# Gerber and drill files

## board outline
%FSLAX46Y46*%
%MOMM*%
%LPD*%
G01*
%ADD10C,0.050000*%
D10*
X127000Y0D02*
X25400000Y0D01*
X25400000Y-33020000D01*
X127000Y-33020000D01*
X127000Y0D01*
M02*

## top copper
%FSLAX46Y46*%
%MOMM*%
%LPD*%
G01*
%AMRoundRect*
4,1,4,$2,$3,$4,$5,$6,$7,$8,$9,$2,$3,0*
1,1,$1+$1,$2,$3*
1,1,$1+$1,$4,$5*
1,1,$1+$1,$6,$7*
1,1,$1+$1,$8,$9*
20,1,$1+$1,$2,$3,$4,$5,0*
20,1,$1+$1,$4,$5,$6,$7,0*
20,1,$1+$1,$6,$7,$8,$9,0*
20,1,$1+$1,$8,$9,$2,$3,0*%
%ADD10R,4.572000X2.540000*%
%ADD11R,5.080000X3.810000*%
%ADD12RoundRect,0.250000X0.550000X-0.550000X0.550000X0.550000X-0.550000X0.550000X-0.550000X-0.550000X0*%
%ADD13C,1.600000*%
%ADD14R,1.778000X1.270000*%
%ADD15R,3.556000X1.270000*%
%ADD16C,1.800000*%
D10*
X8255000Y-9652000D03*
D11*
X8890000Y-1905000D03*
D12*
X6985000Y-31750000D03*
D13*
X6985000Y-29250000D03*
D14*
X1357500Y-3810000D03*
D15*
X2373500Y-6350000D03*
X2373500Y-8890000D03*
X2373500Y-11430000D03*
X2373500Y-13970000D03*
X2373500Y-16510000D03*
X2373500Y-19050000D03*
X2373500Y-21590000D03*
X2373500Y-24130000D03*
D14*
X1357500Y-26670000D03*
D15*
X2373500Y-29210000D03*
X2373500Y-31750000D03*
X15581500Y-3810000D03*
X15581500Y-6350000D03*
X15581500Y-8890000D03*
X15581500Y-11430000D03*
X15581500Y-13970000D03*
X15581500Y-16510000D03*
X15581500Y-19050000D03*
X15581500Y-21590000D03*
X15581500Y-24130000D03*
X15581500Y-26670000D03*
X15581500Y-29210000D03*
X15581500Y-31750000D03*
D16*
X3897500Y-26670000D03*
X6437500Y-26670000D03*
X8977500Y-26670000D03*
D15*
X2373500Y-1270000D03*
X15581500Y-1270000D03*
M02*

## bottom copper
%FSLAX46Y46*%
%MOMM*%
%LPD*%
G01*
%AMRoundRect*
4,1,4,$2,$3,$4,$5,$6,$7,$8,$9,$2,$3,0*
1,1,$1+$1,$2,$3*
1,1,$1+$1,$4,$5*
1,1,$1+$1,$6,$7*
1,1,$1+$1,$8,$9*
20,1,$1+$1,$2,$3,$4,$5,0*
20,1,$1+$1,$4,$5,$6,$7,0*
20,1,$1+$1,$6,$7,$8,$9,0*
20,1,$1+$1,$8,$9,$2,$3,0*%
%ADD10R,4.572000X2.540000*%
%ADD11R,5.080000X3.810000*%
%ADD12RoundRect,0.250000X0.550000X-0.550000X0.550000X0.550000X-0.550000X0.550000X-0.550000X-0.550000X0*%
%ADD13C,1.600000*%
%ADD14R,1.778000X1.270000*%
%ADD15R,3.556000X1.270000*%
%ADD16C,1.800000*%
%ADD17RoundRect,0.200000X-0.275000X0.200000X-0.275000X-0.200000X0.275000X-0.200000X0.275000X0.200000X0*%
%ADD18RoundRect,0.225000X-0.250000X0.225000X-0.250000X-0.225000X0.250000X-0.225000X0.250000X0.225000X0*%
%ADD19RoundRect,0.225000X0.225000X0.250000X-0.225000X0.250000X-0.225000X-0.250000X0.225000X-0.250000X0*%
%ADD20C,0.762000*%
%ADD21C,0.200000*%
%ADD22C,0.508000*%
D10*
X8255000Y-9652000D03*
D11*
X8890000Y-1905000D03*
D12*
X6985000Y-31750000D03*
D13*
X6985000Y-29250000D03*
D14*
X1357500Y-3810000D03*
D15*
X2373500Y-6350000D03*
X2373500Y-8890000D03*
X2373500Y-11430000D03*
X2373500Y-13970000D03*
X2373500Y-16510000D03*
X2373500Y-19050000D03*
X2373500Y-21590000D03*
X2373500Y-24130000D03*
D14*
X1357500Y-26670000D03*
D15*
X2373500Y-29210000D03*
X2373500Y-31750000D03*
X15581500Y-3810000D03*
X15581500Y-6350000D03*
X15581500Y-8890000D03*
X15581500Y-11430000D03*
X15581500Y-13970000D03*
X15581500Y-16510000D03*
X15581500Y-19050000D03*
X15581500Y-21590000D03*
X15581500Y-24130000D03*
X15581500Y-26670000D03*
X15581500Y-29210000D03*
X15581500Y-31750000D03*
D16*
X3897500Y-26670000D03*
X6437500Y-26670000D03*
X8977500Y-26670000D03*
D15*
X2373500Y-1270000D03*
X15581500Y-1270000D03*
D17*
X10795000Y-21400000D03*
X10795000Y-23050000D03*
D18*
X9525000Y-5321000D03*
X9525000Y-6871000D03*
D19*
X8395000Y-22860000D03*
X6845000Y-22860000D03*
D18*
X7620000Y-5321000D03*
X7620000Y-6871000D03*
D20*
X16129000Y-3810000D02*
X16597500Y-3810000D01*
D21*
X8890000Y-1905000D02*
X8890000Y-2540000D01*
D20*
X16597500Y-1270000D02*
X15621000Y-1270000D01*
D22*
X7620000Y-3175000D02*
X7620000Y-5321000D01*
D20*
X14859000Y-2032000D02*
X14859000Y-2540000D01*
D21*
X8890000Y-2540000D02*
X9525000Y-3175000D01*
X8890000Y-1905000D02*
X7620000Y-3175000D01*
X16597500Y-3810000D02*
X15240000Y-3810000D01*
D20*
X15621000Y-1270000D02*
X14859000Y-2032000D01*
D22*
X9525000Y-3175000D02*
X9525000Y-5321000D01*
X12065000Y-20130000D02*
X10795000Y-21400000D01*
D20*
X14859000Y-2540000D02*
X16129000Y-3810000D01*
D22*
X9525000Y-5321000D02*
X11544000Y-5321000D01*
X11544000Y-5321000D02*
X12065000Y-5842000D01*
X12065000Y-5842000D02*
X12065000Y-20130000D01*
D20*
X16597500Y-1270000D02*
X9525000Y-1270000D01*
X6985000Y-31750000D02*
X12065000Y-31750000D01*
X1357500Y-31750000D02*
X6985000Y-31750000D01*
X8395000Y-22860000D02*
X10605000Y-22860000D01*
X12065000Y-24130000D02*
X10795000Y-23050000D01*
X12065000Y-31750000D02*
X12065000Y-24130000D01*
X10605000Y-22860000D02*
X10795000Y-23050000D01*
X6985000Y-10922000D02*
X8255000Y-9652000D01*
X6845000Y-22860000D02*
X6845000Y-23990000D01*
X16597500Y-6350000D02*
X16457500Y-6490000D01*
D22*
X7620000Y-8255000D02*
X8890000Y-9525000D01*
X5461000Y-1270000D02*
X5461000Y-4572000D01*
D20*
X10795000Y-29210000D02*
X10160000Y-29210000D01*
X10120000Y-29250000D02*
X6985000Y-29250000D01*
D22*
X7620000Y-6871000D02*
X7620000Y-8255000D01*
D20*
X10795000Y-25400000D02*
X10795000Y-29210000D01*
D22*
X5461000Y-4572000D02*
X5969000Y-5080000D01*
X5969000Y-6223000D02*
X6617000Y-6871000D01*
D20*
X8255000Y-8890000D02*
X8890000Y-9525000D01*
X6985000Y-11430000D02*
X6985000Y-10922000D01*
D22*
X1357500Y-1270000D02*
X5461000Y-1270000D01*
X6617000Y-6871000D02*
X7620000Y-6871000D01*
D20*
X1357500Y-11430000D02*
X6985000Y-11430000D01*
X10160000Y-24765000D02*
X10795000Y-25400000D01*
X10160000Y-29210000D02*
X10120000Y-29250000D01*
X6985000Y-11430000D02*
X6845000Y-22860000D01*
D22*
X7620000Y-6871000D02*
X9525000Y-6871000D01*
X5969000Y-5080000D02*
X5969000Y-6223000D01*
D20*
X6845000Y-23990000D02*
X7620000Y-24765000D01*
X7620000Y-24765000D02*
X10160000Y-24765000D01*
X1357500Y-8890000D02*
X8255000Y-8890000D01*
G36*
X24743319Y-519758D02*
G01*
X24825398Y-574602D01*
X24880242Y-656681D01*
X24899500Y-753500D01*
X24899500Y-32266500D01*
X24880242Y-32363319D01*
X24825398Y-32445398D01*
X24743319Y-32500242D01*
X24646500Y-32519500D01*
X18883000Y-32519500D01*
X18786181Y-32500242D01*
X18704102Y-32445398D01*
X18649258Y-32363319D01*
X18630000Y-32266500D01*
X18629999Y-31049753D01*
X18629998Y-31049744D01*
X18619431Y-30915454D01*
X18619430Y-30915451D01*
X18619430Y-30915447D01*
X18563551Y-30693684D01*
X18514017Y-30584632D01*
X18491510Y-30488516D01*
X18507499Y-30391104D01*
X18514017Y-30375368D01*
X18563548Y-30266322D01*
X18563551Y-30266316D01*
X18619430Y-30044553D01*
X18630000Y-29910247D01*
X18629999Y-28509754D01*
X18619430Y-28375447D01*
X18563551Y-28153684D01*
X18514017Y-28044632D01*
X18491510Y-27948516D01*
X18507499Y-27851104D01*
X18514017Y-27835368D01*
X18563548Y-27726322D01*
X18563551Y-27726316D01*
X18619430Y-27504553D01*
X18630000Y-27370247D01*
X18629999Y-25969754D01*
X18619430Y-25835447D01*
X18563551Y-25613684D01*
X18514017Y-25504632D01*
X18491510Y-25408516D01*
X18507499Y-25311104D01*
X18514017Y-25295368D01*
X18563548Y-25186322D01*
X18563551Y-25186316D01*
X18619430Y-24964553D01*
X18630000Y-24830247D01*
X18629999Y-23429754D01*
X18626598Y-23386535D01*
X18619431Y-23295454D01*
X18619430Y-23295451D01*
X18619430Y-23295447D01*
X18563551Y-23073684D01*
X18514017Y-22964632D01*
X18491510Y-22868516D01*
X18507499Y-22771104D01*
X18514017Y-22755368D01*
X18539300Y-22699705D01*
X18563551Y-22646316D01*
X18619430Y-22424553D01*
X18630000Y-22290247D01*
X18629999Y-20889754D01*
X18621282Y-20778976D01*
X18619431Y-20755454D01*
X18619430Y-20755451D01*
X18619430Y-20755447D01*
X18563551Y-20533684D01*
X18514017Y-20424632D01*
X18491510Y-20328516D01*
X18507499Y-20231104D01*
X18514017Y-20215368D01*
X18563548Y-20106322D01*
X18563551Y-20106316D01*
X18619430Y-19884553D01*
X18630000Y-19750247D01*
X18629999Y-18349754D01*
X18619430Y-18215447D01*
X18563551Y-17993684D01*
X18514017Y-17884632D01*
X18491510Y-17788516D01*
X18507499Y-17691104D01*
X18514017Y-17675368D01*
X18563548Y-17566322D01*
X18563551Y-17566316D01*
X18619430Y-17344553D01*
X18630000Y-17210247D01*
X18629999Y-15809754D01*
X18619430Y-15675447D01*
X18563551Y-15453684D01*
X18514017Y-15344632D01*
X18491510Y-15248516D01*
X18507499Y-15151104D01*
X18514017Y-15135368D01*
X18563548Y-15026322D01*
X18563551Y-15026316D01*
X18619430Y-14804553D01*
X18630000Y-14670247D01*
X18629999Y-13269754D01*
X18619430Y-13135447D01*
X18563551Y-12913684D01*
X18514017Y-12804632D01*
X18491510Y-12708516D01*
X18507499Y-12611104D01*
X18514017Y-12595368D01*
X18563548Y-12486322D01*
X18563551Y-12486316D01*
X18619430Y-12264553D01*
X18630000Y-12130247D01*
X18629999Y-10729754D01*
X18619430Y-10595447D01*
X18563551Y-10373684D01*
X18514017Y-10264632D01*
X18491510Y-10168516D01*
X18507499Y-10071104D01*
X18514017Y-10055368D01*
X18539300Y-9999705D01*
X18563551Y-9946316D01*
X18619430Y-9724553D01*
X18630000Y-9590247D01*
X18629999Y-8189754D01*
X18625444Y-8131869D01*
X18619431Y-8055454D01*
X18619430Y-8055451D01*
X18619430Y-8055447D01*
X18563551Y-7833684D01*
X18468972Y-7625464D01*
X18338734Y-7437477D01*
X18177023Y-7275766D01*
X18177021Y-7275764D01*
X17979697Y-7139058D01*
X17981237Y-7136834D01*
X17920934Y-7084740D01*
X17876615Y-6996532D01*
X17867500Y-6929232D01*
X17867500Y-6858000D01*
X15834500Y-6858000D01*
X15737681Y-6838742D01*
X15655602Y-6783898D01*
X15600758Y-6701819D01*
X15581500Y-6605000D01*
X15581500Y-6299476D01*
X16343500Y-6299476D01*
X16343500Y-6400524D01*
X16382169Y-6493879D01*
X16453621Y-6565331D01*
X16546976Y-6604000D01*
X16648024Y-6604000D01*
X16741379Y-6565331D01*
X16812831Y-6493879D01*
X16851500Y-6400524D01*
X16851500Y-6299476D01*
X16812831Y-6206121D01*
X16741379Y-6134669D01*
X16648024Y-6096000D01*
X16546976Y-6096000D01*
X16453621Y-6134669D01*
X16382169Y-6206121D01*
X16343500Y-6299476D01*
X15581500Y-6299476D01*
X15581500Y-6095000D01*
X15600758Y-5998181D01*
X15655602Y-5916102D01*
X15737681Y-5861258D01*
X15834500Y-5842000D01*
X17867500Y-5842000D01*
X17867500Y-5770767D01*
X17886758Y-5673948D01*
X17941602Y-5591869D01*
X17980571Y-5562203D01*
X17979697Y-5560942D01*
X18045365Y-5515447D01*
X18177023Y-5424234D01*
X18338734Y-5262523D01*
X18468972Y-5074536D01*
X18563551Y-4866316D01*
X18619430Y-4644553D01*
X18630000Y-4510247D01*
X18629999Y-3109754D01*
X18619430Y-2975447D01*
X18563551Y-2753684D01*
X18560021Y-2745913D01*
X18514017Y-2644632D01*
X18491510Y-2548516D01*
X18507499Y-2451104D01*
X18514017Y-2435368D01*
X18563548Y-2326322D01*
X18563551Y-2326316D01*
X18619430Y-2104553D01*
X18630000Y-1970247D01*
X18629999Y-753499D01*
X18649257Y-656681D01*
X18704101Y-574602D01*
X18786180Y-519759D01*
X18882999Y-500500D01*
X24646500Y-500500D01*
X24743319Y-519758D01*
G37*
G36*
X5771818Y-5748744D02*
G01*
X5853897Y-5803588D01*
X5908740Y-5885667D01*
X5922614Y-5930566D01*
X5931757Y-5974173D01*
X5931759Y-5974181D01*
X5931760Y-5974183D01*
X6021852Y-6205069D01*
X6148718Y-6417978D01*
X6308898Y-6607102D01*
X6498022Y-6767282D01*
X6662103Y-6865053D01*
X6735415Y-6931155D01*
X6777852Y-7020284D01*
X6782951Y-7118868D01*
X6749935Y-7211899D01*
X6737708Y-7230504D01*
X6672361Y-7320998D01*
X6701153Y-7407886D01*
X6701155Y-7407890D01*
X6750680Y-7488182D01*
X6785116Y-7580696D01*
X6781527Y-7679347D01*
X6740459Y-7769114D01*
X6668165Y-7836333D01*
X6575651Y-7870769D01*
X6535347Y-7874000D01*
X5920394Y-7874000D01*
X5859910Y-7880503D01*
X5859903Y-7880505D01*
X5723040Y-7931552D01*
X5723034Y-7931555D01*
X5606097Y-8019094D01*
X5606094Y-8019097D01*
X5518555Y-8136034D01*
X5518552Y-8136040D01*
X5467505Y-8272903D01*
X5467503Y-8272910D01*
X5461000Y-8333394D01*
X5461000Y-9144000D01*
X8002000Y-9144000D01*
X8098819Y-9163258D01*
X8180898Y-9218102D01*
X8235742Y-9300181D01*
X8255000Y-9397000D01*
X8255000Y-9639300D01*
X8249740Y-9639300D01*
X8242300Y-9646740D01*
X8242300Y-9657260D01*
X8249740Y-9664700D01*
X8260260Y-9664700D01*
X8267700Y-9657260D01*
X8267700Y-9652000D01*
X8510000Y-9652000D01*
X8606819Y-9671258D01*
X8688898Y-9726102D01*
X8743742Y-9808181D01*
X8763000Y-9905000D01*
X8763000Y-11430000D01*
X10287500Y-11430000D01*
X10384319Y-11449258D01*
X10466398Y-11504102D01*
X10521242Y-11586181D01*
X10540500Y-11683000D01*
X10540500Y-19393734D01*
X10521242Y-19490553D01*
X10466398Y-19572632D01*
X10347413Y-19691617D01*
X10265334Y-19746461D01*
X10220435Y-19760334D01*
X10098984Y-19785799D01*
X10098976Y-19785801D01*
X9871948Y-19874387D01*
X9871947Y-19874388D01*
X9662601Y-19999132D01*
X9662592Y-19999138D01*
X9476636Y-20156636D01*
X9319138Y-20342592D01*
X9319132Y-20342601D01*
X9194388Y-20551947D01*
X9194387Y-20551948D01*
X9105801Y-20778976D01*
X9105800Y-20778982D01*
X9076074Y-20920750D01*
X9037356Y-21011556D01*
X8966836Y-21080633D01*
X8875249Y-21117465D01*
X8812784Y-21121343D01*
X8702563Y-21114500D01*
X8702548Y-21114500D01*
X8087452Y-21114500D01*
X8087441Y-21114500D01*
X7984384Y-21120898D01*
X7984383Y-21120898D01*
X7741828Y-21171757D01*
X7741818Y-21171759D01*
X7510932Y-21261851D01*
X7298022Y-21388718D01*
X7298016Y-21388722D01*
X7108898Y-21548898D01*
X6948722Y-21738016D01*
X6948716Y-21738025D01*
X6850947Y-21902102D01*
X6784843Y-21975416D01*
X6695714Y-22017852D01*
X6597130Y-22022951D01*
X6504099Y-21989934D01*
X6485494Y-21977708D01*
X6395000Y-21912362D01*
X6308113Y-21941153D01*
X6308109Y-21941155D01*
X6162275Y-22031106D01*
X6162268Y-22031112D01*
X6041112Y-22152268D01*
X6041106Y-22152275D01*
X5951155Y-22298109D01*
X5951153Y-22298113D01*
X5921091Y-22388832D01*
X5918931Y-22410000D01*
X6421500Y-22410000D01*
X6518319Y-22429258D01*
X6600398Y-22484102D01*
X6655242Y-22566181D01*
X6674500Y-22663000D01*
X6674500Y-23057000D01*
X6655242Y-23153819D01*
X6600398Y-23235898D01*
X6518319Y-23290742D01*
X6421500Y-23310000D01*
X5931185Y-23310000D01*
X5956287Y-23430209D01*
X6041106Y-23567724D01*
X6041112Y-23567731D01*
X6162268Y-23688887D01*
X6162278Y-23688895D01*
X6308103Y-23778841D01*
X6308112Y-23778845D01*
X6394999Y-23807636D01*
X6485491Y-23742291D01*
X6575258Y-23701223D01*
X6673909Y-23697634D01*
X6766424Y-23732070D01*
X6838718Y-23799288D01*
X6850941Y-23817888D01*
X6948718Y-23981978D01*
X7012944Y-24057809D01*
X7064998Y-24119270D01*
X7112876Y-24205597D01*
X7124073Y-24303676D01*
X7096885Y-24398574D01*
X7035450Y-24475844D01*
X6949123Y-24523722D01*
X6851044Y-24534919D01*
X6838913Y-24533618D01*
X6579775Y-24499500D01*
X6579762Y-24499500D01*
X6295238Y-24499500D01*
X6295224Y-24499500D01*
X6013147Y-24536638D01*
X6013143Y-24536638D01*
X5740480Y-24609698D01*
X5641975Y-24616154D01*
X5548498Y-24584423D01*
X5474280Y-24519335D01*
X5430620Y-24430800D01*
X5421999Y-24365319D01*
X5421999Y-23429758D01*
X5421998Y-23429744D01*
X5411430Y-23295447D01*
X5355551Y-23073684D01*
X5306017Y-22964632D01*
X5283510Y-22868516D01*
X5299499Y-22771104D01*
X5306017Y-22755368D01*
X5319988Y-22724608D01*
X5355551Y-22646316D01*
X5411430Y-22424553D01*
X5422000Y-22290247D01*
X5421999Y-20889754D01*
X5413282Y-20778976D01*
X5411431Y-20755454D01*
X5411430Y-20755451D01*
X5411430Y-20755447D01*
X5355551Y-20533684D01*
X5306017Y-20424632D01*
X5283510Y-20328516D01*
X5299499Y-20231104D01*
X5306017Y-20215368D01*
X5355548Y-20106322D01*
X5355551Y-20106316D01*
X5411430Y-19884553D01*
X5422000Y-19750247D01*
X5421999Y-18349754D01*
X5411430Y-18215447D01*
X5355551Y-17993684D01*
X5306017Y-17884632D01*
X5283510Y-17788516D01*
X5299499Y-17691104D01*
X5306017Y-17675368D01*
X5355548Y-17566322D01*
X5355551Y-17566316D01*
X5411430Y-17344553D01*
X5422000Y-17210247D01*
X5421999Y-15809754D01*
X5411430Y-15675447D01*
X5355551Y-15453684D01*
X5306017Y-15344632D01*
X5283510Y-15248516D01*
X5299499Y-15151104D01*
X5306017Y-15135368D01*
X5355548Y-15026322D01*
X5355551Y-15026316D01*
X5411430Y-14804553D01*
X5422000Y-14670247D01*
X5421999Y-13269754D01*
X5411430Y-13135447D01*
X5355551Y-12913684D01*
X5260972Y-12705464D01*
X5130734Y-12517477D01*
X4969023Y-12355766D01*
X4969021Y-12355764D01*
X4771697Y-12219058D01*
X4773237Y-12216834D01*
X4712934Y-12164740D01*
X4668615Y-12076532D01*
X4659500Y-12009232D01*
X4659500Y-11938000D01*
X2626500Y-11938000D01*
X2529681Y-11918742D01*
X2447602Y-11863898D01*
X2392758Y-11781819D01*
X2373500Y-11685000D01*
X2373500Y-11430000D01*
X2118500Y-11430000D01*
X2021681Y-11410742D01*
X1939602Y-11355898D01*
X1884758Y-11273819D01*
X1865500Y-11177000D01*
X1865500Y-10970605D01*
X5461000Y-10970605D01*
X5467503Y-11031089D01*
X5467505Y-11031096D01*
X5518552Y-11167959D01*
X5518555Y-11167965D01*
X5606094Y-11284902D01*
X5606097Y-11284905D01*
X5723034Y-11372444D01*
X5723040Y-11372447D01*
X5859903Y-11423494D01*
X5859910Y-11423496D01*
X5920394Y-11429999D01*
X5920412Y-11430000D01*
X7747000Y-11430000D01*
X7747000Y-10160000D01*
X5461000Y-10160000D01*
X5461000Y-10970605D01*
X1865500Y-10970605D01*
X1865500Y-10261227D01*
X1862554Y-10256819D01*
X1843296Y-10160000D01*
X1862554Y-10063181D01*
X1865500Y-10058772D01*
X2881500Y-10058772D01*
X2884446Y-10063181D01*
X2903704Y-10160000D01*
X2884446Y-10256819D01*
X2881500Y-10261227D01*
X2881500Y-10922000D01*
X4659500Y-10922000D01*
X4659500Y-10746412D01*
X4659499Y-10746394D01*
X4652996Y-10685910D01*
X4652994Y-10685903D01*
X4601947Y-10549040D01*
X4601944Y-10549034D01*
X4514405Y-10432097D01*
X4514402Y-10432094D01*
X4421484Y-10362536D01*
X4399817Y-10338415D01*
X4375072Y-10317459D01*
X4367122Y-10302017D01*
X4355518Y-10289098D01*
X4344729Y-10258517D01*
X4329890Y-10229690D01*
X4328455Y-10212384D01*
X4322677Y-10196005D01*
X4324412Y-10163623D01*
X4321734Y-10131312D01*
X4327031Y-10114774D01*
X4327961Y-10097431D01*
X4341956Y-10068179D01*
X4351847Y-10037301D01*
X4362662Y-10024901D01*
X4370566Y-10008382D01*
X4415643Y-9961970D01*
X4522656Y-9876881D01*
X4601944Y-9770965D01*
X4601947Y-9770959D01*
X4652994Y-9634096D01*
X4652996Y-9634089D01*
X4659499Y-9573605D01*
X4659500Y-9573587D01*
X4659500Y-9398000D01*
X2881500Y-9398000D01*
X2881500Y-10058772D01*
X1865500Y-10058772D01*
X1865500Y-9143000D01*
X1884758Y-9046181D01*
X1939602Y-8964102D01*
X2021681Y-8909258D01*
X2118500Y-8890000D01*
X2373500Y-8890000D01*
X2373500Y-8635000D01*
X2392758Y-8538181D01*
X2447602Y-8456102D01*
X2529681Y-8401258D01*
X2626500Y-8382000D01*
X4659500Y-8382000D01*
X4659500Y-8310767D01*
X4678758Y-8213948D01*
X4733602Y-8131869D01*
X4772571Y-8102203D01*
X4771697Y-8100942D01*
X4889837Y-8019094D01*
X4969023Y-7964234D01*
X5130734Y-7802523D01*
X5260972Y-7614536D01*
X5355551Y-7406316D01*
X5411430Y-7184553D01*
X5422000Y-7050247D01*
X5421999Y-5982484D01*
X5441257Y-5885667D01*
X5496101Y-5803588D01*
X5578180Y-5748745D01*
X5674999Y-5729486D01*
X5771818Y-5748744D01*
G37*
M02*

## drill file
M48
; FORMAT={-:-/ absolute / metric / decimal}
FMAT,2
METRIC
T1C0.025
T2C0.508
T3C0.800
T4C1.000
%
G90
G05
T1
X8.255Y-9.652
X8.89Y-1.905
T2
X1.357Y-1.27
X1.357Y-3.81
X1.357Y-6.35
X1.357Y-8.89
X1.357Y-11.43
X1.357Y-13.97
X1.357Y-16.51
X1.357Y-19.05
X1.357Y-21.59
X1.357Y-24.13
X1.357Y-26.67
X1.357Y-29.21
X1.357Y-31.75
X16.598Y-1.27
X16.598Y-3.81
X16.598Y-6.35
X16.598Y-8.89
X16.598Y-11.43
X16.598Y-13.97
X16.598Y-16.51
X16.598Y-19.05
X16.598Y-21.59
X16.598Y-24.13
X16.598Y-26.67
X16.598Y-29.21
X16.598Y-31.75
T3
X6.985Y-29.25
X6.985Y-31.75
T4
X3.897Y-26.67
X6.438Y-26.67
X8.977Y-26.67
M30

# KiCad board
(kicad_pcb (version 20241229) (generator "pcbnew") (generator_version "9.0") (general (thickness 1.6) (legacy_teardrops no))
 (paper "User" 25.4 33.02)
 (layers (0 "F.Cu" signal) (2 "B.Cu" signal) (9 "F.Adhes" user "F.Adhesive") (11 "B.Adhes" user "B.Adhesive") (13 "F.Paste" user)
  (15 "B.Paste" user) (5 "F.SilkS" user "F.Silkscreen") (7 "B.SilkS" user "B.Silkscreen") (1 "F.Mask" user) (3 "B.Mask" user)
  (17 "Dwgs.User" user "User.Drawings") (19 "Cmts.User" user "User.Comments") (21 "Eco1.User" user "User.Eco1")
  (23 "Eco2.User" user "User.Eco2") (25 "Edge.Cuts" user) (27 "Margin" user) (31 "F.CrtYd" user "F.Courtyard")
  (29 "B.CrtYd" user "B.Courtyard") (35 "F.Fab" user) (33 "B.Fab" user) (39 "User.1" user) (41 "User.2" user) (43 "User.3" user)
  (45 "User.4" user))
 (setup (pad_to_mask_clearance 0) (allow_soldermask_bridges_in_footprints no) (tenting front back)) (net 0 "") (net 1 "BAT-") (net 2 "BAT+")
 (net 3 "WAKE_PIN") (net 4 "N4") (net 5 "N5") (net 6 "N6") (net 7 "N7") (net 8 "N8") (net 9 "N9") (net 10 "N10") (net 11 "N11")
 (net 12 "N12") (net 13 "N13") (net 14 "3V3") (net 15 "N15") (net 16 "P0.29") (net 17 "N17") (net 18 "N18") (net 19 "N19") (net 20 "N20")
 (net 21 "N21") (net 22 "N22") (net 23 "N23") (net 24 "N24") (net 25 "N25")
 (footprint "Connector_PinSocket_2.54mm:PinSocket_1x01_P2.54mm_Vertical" (layer "F.Cu") (at 8.255 9.652)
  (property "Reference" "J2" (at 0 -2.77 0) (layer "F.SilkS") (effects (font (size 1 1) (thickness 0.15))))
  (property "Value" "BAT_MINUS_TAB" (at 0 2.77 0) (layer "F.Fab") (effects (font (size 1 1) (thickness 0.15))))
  (pad "1" thru_hole rect (at 0 0) (size 4.572 2.54) (drill 0.0254) (layers "*.Cu" "*.Mask") (remove_unused_layers no) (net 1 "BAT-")))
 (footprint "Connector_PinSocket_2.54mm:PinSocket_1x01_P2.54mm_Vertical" (layer "F.Cu") (at 8.89 1.905 180)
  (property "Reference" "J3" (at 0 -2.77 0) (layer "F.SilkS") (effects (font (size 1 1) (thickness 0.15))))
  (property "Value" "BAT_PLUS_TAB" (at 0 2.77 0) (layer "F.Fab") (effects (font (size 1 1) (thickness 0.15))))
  (pad "1" thru_hole rect (at 0 0 180) (size 5.08 3.81) (drill 0.0254) (layers "*.Cu" "*.Mask") (remove_unused_layers no) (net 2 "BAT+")))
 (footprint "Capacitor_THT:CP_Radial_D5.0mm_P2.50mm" (layer "F.Cu") (at 6.985 31.75 90)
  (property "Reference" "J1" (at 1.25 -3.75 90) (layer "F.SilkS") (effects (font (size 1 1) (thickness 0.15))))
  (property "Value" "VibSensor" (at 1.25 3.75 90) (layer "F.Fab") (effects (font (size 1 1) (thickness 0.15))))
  (pad "1" thru_hole roundrect (at 0 0 90) (size 1.6 1.6) (drill 0.8) (layers "*.Cu" "*.Mask") (remove_unused_layers no)
   (roundrect_rratio 0.15625) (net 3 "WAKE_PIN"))
  (pad "2" thru_hole circle (at 2.5 0 90) (size 1.6 1.6) (drill 0.8) (layers "*.Cu" "*.Mask") (remove_unused_layers no) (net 1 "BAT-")))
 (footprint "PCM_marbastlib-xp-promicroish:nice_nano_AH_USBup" (layer "F.Cu") (at 8.9775 17.78)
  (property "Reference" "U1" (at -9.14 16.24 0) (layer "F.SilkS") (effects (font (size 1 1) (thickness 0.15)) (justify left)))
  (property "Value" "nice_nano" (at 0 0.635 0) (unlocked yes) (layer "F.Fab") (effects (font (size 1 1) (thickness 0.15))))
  (pad "1" thru_hole rect (at -7.62 -13.97) (size 1.778 1.27) (drill 0.508) (layers "*.Cu" "B.Mask") (remove_unused_layers no) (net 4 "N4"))
  (pad "2" thru_hole rect (at -7.62 -11.43) (size 3.556 1.27) (drill 0.508 (offset 1.016 0)) (layers "*.Cu" "B.Mask")
   (remove_unused_layers no) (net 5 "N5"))
  (pad "3" thru_hole rect (at -7.62 -8.89) (size 3.556 1.27) (drill 0.508 (offset 1.016 0)) (layers "*.Cu" "B.Mask")
   (remove_unused_layers no) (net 1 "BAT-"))
  (pad "4" thru_hole rect (at -7.62 -6.35) (size 3.556 1.27) (drill 0.508 (offset 1.016 0)) (layers "*.Cu" "B.Mask")
   (remove_unused_layers no) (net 1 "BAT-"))
  (pad "5" thru_hole rect (at -7.62 -3.81) (size 3.556 1.27) (drill 0.508 (offset 1.016 0)) (layers "*.Cu" "B.Mask")
   (remove_unused_layers no) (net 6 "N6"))
  (pad "6" thru_hole rect (at -7.62 -1.27) (size 3.556 1.27) (drill 0.508 (offset 1.016 0)) (layers "*.Cu" "B.Mask")
   (remove_unused_layers no) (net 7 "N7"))
  (pad "7" thru_hole rect (at -7.62 1.27) (size 3.556 1.27) (drill 0.508 (offset 1.016 0)) (layers "*.Cu" "B.Mask")
   (remove_unused_layers no) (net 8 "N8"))
  (pad "8" thru_hole rect (at -7.62 3.81) (size 3.556 1.27) (drill 0.508 (offset 1.016 0)) (layers "*.Cu" "B.Mask")
   (remove_unused_layers no) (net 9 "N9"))
  (pad "9" thru_hole rect (at -7.62 6.35) (size 3.556 1.27) (drill 0.508 (offset 1.016 0)) (layers "*.Cu" "B.Mask")
   (remove_unused_layers no) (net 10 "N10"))
  (pad "10" thru_hole rect (at -7.62 8.89) (size 1.778 1.27) (drill 0.508) (layers "*.Cu" "B.Mask") (remove_unused_layers no) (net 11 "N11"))
  (pad "11" thru_hole rect (at -7.62 11.43) (size 3.556 1.27) (drill 0.508 (offset 1.016 0)) (layers "*.Cu" "B.Mask")
   (remove_unused_layers no) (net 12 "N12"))
  (pad "12" thru_hole rect (at -7.62 13.97) (size 3.556 1.27) (drill 0.508 (offset 1.016 0)) (layers "*.Cu" "B.Mask")
   (remove_unused_layers no) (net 3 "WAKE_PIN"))
  (pad "13" thru_hole rect (at 7.62 -13.97) (size 3.556 1.27) (drill 0.508 (offset -1.016 0)) (layers "*.Cu" "B.Mask")
   (remove_unused_layers no) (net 2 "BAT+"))
  (pad "14" thru_hole rect (at 7.62 -11.43) (size 3.556 1.27) (drill 0.508 (offset -1.016 0)) (layers "*.Cu" "B.Mask")
   (remove_unused_layers no) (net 1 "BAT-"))
  (pad "15" thru_hole rect (at 7.62 -8.89) (size 3.556 1.27) (drill 0.508 (offset -1.016 0)) (layers "*.Cu" "B.Mask")
   (remove_unused_layers no) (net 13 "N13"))
  (pad "16" thru_hole rect (at 7.62 -6.35) (size 3.556 1.27) (drill 0.508 (offset -1.016 0)) (layers "*.Cu" "B.Mask")
   (remove_unused_layers no) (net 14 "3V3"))
  (pad "17" thru_hole rect (at 7.62 -3.81) (size 3.556 1.27) (drill 0.508 (offset -1.016 0)) (layers "*.Cu" "B.Mask")
   (remove_unused_layers no) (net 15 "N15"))
  (pad "18" thru_hole rect (at 7.62 -1.27) (size 3.556 1.27) (drill 0.508 (offset -1.016 0)) (layers "*.Cu" "B.Mask")
   (remove_unused_layers no) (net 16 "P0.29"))
  (pad "19" thru_hole rect (at 7.62 1.27) (size 3.556 1.27) (drill 0.508 (offset -1.016 0)) (layers "*.Cu" "B.Mask")
   (remove_unused_layers no) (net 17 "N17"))
  (pad "20" thru_hole rect (at 7.62 3.81) (size 3.556 1.27) (drill 0.508 (offset -1.016 0)) (layers "*.Cu" "B.Mask")
   (remove_unused_layers no) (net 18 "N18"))
  (pad "21" thru_hole rect (at 7.62 6.35) (size 3.556 1.27) (drill 0.508 (offset -1.016 0)) (layers "*.Cu" "B.Mask")
   (remove_unused_layers no) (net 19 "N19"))
  (pad "22" thru_hole rect (at 7.62 8.89) (size 3.556 1.27) (drill 0.508 (offset -1.016 0)) (layers "*.Cu" "B.Mask")
   (remove_unused_layers no) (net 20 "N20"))
  (pad "23" thru_hole rect (at 7.62 11.43) (size 3.556 1.27) (drill 0.508 (offset -1.016 0)) (layers "*.Cu" "B.Mask")
   (remove_unused_layers no) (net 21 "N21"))
  (pad "24" thru_hole rect (at 7.62 13.97) (size 3.556 1.27) (drill 0.508 (offset -1.016 0)) (layers "*.Cu" "B.Mask")
   (remove_unused_layers no) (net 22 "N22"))
  (pad "25" thru_hole circle (at -5.08 8.89) (size 1.8 1.8) (drill 1) (layers "*.Cu" "B.Mask") (remove_unused_layers no) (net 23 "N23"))
  (pad "26" thru_hole circle (at -2.54 8.89) (size 1.8 1.8) (drill 1) (layers "*.Cu" "B.Mask") (remove_unused_layers no) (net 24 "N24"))
  (pad "27" thru_hole circle (at 0 8.89) (size 1.8 1.8) (drill 1) (layers "*.Cu" "B.Mask") (remove_unused_layers no) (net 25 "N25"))
  (pad "28" thru_hole rect (at -7.62 -16.51) (size 3.556 1.27) (drill 0.508 (offset 1.016 0)) (layers "*.Cu" "B.Mask")
   (remove_unused_layers no) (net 1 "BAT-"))
  (pad "29" thru_hole rect (at 7.62 -16.51) (size 3.556 1.27) (drill 0.508 (offset -1.016 0)) (layers "*.Cu" "B.Mask")
   (remove_unused_layers no) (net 2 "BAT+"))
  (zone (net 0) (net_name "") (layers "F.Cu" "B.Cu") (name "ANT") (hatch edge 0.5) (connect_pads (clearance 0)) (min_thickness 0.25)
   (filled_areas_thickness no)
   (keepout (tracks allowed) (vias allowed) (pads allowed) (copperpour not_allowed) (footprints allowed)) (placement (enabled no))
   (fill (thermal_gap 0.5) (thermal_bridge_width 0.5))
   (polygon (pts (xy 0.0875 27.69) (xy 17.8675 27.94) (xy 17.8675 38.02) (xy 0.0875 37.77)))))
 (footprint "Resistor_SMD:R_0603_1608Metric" (layer "B.Cu") (at 10.795 22.225 -90)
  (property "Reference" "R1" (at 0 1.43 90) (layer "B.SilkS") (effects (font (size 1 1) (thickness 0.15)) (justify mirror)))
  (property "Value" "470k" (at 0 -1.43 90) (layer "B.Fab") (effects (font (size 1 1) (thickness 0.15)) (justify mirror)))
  (pad "1" smd roundrect (at -0.825 0 270) (size 0.8 0.95) (layers "B.Cu" "B.Mask" "B.Paste") (roundrect_rratio 0.25) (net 2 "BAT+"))
  (pad "2" smd roundrect (at 0.825 0 270) (size 0.8 0.95) (layers "B.Cu" "B.Mask" "B.Paste") (roundrect_rratio 0.25) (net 3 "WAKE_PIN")))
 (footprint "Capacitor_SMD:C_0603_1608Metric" (layer "B.Cu") (at 9.525 6.096 -90)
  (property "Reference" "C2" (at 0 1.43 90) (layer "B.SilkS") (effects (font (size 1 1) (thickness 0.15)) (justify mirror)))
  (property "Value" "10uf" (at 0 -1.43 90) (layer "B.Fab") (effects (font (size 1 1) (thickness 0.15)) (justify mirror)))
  (pad "1" smd roundrect (at -0.775 0 270) (size 0.9 0.95) (layers "B.Cu" "B.Mask" "B.Paste") (roundrect_rratio 0.25) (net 2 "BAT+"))
  (pad "2" smd roundrect (at 0.775 0 270) (size 0.9 0.95) (layers "B.Cu" "B.Mask" "B.Paste") (roundrect_rratio 0.25) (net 1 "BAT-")))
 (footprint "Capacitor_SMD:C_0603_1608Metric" (layer "B.Cu") (at 7.62 22.86 180)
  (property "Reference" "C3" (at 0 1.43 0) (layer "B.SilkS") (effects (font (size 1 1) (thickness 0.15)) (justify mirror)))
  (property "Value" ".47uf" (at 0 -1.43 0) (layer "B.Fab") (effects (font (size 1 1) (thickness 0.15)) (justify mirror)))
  (pad "1" smd roundrect (at -0.775 0 180) (size 0.9 0.95) (layers "B.Cu" "B.Mask" "B.Paste") (roundrect_rratio 0.25) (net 3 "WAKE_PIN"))
  (pad "2" smd roundrect (at 0.775 0 180) (size 0.9 0.95) (layers "B.Cu" "B.Mask" "B.Paste") (roundrect_rratio 0.25) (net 1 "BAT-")))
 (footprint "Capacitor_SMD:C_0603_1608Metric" (layer "B.Cu") (at 7.62 6.096 -90)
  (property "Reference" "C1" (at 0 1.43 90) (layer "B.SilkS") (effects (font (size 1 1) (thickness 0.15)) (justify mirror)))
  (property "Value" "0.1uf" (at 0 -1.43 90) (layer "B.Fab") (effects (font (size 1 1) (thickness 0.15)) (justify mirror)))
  (pad "1" smd roundrect (at -0.775 0 270) (size 0.9 0.95) (layers "B.Cu" "B.Mask" "B.Paste") (roundrect_rratio 0.25) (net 2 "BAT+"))
  (pad "2" smd roundrect (at 0.775 0 270) (size 0.9 0.95) (layers "B.Cu" "B.Mask" "B.Paste") (roundrect_rratio 0.25) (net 1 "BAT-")))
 (gr_rect (start 0.127 0) (end 25.4 33.02) (stroke (width 0.05) (type default)) (fill no) (layer "Edge.Cuts"))
 (segment (start 16.129 3.81) (end 16.5975 3.81) (width 0.762) (layer "B.Cu") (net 2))
 (segment (start 8.89 1.905) (end 8.89 2.54) (width 0.2) (layer "B.Cu") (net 2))
 (segment (start 16.5975 1.27) (end 15.621 1.27) (width 0.762) (layer "B.Cu") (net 2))
 (segment (start 7.62 3.175) (end 7.62 5.321) (width 0.508) (layer "B.Cu") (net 2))
 (segment (start 14.859 2.032) (end 14.859 2.54) (width 0.762) (layer "B.Cu") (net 2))
 (segment (start 8.89 2.54) (end 9.525 3.175) (width 0.2) (layer "B.Cu") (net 2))
 (segment (start 8.89 1.905) (end 7.62 3.175) (width 0.2) (layer "B.Cu") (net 2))
 (segment (start 16.5975 3.81) (end 15.24 3.81) (width 0.2) (layer "B.Cu") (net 2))
 (segment (start 15.621 1.27) (end 14.859 2.032) (width 0.762) (layer "B.Cu") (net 2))
 (segment (start 9.525 3.175) (end 9.525 5.321) (width 0.508) (layer "B.Cu") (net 2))
 (segment (start 12.065 20.13) (end 10.795 21.4) (width 0.508) (layer "B.Cu") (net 2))
 (segment (start 14.859 2.54) (end 16.129 3.81) (width 0.762) (layer "B.Cu") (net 2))
 (segment (start 9.525 5.321) (end 11.544 5.321) (width 0.508) (layer "B.Cu") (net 2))
 (segment (start 11.544 5.321) (end 12.065 5.842) (width 0.508) (layer "B.Cu") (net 2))
 (segment (start 12.065 5.842) (end 12.065 20.13) (width 0.508) (layer "B.Cu") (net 2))
 (segment (start 16.5975 1.27) (end 9.525 1.27) (width 0.762) (layer "B.Cu") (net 2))
 (segment (start 6.985 31.75) (end 12.065 31.75) (width 0.762) (layer "B.Cu") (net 3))
 (segment (start 1.3575 31.75) (end 6.985 31.75) (width 0.762) (layer "B.Cu") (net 3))
 (segment (start 8.395 22.86) (end 10.605 22.86) (width 0.762) (layer "B.Cu") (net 3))
 (segment (start 12.065 24.13) (end 10.795 23.05) (width 0.762) (layer "B.Cu") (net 3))
 (segment (start 12.065 31.75) (end 12.065 24.13) (width 0.762) (layer "B.Cu") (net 3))
 (segment (start 10.605 22.86) (end 10.795 23.05) (width 0.762) (layer "B.Cu") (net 3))
 (segment (start 6.985 10.922) (end 8.255 9.652) (width 0.762) (layer "B.Cu") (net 1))
 (segment (start 6.845 22.86) (end 6.845 23.99) (width 0.762) (layer "B.Cu") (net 1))
 (segment (start 16.5975 6.35) (end 16.4575 6.49) (width 0.762) (layer "B.Cu") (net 1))
 (segment (start 7.62 8.255) (end 8.89 9.525) (width 0.508) (layer "B.Cu") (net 1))
 (segment (start 5.461 1.27) (end 5.461 4.572) (width 0.508) (layer "B.Cu") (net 1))
 (segment (start 10.795 29.21) (end 10.16 29.21) (width 0.762) (layer "B.Cu") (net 1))
 (segment (start 10.12 29.25) (end 6.985 29.25) (width 0.762) (layer "B.Cu") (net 1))
 (segment (start 7.62 6.871) (end 7.62 8.255) (width 0.508) (layer "B.Cu") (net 1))
 (segment (start 10.795 25.4) (end 10.795 29.21) (width 0.762) (layer "B.Cu") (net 1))
 (segment (start 5.461 4.572) (end 5.969 5.08) (width 0.508) (layer "B.Cu") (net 1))
 (segment (start 5.969 6.223) (end 6.617 6.871) (width 0.508) (layer "B.Cu") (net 1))
 (segment (start 8.255 8.89) (end 8.89 9.525) (width 0.762) (layer "B.Cu") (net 1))
 (segment (start 6.985 11.43) (end 6.985 10.922) (width 0.762) (layer "B.Cu") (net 1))
 (segment (start 1.3575 1.27) (end 5.461 1.27) (width 0.508) (layer "B.Cu") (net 1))
 (segment (start 6.617 6.871) (end 7.62 6.871) (width 0.508) (layer "B.Cu") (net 1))
 (segment (start 1.3575 11.43) (end 6.985 11.43) (width 0.762) (layer "B.Cu") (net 1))
 (segment (start 10.16 24.765) (end 10.795 25.4) (width 0.762) (layer "B.Cu") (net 1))
 (segment (start 10.16 29.21) (end 10.12 29.25) (width 0.762) (layer "B.Cu") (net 1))
 (segment (start 6.985 11.43) (end 6.845 22.86) (width 0.762) (layer "B.Cu") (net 1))
 (segment (start 7.62 6.871) (end 9.525 6.871) (width 0.508) (layer "B.Cu") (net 1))
 (segment (start 5.969 5.08) (end 5.969 6.223) (width 0.508) (layer "B.Cu") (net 1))
 (segment (start 6.845 23.99) (end 7.62 24.765) (width 0.762) (layer "B.Cu") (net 1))
 (segment (start 7.62 24.765) (end 10.16 24.765) (width 0.762) (layer "B.Cu") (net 1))
 (segment (start 1.3575 8.89) (end 8.255 8.89) (width 0.762) (layer "B.Cu") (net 1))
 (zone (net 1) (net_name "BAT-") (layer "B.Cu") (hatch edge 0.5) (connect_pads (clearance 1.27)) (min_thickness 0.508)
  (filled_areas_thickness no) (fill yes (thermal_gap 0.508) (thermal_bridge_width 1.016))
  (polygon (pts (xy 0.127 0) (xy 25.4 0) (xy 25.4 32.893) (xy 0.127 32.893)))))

